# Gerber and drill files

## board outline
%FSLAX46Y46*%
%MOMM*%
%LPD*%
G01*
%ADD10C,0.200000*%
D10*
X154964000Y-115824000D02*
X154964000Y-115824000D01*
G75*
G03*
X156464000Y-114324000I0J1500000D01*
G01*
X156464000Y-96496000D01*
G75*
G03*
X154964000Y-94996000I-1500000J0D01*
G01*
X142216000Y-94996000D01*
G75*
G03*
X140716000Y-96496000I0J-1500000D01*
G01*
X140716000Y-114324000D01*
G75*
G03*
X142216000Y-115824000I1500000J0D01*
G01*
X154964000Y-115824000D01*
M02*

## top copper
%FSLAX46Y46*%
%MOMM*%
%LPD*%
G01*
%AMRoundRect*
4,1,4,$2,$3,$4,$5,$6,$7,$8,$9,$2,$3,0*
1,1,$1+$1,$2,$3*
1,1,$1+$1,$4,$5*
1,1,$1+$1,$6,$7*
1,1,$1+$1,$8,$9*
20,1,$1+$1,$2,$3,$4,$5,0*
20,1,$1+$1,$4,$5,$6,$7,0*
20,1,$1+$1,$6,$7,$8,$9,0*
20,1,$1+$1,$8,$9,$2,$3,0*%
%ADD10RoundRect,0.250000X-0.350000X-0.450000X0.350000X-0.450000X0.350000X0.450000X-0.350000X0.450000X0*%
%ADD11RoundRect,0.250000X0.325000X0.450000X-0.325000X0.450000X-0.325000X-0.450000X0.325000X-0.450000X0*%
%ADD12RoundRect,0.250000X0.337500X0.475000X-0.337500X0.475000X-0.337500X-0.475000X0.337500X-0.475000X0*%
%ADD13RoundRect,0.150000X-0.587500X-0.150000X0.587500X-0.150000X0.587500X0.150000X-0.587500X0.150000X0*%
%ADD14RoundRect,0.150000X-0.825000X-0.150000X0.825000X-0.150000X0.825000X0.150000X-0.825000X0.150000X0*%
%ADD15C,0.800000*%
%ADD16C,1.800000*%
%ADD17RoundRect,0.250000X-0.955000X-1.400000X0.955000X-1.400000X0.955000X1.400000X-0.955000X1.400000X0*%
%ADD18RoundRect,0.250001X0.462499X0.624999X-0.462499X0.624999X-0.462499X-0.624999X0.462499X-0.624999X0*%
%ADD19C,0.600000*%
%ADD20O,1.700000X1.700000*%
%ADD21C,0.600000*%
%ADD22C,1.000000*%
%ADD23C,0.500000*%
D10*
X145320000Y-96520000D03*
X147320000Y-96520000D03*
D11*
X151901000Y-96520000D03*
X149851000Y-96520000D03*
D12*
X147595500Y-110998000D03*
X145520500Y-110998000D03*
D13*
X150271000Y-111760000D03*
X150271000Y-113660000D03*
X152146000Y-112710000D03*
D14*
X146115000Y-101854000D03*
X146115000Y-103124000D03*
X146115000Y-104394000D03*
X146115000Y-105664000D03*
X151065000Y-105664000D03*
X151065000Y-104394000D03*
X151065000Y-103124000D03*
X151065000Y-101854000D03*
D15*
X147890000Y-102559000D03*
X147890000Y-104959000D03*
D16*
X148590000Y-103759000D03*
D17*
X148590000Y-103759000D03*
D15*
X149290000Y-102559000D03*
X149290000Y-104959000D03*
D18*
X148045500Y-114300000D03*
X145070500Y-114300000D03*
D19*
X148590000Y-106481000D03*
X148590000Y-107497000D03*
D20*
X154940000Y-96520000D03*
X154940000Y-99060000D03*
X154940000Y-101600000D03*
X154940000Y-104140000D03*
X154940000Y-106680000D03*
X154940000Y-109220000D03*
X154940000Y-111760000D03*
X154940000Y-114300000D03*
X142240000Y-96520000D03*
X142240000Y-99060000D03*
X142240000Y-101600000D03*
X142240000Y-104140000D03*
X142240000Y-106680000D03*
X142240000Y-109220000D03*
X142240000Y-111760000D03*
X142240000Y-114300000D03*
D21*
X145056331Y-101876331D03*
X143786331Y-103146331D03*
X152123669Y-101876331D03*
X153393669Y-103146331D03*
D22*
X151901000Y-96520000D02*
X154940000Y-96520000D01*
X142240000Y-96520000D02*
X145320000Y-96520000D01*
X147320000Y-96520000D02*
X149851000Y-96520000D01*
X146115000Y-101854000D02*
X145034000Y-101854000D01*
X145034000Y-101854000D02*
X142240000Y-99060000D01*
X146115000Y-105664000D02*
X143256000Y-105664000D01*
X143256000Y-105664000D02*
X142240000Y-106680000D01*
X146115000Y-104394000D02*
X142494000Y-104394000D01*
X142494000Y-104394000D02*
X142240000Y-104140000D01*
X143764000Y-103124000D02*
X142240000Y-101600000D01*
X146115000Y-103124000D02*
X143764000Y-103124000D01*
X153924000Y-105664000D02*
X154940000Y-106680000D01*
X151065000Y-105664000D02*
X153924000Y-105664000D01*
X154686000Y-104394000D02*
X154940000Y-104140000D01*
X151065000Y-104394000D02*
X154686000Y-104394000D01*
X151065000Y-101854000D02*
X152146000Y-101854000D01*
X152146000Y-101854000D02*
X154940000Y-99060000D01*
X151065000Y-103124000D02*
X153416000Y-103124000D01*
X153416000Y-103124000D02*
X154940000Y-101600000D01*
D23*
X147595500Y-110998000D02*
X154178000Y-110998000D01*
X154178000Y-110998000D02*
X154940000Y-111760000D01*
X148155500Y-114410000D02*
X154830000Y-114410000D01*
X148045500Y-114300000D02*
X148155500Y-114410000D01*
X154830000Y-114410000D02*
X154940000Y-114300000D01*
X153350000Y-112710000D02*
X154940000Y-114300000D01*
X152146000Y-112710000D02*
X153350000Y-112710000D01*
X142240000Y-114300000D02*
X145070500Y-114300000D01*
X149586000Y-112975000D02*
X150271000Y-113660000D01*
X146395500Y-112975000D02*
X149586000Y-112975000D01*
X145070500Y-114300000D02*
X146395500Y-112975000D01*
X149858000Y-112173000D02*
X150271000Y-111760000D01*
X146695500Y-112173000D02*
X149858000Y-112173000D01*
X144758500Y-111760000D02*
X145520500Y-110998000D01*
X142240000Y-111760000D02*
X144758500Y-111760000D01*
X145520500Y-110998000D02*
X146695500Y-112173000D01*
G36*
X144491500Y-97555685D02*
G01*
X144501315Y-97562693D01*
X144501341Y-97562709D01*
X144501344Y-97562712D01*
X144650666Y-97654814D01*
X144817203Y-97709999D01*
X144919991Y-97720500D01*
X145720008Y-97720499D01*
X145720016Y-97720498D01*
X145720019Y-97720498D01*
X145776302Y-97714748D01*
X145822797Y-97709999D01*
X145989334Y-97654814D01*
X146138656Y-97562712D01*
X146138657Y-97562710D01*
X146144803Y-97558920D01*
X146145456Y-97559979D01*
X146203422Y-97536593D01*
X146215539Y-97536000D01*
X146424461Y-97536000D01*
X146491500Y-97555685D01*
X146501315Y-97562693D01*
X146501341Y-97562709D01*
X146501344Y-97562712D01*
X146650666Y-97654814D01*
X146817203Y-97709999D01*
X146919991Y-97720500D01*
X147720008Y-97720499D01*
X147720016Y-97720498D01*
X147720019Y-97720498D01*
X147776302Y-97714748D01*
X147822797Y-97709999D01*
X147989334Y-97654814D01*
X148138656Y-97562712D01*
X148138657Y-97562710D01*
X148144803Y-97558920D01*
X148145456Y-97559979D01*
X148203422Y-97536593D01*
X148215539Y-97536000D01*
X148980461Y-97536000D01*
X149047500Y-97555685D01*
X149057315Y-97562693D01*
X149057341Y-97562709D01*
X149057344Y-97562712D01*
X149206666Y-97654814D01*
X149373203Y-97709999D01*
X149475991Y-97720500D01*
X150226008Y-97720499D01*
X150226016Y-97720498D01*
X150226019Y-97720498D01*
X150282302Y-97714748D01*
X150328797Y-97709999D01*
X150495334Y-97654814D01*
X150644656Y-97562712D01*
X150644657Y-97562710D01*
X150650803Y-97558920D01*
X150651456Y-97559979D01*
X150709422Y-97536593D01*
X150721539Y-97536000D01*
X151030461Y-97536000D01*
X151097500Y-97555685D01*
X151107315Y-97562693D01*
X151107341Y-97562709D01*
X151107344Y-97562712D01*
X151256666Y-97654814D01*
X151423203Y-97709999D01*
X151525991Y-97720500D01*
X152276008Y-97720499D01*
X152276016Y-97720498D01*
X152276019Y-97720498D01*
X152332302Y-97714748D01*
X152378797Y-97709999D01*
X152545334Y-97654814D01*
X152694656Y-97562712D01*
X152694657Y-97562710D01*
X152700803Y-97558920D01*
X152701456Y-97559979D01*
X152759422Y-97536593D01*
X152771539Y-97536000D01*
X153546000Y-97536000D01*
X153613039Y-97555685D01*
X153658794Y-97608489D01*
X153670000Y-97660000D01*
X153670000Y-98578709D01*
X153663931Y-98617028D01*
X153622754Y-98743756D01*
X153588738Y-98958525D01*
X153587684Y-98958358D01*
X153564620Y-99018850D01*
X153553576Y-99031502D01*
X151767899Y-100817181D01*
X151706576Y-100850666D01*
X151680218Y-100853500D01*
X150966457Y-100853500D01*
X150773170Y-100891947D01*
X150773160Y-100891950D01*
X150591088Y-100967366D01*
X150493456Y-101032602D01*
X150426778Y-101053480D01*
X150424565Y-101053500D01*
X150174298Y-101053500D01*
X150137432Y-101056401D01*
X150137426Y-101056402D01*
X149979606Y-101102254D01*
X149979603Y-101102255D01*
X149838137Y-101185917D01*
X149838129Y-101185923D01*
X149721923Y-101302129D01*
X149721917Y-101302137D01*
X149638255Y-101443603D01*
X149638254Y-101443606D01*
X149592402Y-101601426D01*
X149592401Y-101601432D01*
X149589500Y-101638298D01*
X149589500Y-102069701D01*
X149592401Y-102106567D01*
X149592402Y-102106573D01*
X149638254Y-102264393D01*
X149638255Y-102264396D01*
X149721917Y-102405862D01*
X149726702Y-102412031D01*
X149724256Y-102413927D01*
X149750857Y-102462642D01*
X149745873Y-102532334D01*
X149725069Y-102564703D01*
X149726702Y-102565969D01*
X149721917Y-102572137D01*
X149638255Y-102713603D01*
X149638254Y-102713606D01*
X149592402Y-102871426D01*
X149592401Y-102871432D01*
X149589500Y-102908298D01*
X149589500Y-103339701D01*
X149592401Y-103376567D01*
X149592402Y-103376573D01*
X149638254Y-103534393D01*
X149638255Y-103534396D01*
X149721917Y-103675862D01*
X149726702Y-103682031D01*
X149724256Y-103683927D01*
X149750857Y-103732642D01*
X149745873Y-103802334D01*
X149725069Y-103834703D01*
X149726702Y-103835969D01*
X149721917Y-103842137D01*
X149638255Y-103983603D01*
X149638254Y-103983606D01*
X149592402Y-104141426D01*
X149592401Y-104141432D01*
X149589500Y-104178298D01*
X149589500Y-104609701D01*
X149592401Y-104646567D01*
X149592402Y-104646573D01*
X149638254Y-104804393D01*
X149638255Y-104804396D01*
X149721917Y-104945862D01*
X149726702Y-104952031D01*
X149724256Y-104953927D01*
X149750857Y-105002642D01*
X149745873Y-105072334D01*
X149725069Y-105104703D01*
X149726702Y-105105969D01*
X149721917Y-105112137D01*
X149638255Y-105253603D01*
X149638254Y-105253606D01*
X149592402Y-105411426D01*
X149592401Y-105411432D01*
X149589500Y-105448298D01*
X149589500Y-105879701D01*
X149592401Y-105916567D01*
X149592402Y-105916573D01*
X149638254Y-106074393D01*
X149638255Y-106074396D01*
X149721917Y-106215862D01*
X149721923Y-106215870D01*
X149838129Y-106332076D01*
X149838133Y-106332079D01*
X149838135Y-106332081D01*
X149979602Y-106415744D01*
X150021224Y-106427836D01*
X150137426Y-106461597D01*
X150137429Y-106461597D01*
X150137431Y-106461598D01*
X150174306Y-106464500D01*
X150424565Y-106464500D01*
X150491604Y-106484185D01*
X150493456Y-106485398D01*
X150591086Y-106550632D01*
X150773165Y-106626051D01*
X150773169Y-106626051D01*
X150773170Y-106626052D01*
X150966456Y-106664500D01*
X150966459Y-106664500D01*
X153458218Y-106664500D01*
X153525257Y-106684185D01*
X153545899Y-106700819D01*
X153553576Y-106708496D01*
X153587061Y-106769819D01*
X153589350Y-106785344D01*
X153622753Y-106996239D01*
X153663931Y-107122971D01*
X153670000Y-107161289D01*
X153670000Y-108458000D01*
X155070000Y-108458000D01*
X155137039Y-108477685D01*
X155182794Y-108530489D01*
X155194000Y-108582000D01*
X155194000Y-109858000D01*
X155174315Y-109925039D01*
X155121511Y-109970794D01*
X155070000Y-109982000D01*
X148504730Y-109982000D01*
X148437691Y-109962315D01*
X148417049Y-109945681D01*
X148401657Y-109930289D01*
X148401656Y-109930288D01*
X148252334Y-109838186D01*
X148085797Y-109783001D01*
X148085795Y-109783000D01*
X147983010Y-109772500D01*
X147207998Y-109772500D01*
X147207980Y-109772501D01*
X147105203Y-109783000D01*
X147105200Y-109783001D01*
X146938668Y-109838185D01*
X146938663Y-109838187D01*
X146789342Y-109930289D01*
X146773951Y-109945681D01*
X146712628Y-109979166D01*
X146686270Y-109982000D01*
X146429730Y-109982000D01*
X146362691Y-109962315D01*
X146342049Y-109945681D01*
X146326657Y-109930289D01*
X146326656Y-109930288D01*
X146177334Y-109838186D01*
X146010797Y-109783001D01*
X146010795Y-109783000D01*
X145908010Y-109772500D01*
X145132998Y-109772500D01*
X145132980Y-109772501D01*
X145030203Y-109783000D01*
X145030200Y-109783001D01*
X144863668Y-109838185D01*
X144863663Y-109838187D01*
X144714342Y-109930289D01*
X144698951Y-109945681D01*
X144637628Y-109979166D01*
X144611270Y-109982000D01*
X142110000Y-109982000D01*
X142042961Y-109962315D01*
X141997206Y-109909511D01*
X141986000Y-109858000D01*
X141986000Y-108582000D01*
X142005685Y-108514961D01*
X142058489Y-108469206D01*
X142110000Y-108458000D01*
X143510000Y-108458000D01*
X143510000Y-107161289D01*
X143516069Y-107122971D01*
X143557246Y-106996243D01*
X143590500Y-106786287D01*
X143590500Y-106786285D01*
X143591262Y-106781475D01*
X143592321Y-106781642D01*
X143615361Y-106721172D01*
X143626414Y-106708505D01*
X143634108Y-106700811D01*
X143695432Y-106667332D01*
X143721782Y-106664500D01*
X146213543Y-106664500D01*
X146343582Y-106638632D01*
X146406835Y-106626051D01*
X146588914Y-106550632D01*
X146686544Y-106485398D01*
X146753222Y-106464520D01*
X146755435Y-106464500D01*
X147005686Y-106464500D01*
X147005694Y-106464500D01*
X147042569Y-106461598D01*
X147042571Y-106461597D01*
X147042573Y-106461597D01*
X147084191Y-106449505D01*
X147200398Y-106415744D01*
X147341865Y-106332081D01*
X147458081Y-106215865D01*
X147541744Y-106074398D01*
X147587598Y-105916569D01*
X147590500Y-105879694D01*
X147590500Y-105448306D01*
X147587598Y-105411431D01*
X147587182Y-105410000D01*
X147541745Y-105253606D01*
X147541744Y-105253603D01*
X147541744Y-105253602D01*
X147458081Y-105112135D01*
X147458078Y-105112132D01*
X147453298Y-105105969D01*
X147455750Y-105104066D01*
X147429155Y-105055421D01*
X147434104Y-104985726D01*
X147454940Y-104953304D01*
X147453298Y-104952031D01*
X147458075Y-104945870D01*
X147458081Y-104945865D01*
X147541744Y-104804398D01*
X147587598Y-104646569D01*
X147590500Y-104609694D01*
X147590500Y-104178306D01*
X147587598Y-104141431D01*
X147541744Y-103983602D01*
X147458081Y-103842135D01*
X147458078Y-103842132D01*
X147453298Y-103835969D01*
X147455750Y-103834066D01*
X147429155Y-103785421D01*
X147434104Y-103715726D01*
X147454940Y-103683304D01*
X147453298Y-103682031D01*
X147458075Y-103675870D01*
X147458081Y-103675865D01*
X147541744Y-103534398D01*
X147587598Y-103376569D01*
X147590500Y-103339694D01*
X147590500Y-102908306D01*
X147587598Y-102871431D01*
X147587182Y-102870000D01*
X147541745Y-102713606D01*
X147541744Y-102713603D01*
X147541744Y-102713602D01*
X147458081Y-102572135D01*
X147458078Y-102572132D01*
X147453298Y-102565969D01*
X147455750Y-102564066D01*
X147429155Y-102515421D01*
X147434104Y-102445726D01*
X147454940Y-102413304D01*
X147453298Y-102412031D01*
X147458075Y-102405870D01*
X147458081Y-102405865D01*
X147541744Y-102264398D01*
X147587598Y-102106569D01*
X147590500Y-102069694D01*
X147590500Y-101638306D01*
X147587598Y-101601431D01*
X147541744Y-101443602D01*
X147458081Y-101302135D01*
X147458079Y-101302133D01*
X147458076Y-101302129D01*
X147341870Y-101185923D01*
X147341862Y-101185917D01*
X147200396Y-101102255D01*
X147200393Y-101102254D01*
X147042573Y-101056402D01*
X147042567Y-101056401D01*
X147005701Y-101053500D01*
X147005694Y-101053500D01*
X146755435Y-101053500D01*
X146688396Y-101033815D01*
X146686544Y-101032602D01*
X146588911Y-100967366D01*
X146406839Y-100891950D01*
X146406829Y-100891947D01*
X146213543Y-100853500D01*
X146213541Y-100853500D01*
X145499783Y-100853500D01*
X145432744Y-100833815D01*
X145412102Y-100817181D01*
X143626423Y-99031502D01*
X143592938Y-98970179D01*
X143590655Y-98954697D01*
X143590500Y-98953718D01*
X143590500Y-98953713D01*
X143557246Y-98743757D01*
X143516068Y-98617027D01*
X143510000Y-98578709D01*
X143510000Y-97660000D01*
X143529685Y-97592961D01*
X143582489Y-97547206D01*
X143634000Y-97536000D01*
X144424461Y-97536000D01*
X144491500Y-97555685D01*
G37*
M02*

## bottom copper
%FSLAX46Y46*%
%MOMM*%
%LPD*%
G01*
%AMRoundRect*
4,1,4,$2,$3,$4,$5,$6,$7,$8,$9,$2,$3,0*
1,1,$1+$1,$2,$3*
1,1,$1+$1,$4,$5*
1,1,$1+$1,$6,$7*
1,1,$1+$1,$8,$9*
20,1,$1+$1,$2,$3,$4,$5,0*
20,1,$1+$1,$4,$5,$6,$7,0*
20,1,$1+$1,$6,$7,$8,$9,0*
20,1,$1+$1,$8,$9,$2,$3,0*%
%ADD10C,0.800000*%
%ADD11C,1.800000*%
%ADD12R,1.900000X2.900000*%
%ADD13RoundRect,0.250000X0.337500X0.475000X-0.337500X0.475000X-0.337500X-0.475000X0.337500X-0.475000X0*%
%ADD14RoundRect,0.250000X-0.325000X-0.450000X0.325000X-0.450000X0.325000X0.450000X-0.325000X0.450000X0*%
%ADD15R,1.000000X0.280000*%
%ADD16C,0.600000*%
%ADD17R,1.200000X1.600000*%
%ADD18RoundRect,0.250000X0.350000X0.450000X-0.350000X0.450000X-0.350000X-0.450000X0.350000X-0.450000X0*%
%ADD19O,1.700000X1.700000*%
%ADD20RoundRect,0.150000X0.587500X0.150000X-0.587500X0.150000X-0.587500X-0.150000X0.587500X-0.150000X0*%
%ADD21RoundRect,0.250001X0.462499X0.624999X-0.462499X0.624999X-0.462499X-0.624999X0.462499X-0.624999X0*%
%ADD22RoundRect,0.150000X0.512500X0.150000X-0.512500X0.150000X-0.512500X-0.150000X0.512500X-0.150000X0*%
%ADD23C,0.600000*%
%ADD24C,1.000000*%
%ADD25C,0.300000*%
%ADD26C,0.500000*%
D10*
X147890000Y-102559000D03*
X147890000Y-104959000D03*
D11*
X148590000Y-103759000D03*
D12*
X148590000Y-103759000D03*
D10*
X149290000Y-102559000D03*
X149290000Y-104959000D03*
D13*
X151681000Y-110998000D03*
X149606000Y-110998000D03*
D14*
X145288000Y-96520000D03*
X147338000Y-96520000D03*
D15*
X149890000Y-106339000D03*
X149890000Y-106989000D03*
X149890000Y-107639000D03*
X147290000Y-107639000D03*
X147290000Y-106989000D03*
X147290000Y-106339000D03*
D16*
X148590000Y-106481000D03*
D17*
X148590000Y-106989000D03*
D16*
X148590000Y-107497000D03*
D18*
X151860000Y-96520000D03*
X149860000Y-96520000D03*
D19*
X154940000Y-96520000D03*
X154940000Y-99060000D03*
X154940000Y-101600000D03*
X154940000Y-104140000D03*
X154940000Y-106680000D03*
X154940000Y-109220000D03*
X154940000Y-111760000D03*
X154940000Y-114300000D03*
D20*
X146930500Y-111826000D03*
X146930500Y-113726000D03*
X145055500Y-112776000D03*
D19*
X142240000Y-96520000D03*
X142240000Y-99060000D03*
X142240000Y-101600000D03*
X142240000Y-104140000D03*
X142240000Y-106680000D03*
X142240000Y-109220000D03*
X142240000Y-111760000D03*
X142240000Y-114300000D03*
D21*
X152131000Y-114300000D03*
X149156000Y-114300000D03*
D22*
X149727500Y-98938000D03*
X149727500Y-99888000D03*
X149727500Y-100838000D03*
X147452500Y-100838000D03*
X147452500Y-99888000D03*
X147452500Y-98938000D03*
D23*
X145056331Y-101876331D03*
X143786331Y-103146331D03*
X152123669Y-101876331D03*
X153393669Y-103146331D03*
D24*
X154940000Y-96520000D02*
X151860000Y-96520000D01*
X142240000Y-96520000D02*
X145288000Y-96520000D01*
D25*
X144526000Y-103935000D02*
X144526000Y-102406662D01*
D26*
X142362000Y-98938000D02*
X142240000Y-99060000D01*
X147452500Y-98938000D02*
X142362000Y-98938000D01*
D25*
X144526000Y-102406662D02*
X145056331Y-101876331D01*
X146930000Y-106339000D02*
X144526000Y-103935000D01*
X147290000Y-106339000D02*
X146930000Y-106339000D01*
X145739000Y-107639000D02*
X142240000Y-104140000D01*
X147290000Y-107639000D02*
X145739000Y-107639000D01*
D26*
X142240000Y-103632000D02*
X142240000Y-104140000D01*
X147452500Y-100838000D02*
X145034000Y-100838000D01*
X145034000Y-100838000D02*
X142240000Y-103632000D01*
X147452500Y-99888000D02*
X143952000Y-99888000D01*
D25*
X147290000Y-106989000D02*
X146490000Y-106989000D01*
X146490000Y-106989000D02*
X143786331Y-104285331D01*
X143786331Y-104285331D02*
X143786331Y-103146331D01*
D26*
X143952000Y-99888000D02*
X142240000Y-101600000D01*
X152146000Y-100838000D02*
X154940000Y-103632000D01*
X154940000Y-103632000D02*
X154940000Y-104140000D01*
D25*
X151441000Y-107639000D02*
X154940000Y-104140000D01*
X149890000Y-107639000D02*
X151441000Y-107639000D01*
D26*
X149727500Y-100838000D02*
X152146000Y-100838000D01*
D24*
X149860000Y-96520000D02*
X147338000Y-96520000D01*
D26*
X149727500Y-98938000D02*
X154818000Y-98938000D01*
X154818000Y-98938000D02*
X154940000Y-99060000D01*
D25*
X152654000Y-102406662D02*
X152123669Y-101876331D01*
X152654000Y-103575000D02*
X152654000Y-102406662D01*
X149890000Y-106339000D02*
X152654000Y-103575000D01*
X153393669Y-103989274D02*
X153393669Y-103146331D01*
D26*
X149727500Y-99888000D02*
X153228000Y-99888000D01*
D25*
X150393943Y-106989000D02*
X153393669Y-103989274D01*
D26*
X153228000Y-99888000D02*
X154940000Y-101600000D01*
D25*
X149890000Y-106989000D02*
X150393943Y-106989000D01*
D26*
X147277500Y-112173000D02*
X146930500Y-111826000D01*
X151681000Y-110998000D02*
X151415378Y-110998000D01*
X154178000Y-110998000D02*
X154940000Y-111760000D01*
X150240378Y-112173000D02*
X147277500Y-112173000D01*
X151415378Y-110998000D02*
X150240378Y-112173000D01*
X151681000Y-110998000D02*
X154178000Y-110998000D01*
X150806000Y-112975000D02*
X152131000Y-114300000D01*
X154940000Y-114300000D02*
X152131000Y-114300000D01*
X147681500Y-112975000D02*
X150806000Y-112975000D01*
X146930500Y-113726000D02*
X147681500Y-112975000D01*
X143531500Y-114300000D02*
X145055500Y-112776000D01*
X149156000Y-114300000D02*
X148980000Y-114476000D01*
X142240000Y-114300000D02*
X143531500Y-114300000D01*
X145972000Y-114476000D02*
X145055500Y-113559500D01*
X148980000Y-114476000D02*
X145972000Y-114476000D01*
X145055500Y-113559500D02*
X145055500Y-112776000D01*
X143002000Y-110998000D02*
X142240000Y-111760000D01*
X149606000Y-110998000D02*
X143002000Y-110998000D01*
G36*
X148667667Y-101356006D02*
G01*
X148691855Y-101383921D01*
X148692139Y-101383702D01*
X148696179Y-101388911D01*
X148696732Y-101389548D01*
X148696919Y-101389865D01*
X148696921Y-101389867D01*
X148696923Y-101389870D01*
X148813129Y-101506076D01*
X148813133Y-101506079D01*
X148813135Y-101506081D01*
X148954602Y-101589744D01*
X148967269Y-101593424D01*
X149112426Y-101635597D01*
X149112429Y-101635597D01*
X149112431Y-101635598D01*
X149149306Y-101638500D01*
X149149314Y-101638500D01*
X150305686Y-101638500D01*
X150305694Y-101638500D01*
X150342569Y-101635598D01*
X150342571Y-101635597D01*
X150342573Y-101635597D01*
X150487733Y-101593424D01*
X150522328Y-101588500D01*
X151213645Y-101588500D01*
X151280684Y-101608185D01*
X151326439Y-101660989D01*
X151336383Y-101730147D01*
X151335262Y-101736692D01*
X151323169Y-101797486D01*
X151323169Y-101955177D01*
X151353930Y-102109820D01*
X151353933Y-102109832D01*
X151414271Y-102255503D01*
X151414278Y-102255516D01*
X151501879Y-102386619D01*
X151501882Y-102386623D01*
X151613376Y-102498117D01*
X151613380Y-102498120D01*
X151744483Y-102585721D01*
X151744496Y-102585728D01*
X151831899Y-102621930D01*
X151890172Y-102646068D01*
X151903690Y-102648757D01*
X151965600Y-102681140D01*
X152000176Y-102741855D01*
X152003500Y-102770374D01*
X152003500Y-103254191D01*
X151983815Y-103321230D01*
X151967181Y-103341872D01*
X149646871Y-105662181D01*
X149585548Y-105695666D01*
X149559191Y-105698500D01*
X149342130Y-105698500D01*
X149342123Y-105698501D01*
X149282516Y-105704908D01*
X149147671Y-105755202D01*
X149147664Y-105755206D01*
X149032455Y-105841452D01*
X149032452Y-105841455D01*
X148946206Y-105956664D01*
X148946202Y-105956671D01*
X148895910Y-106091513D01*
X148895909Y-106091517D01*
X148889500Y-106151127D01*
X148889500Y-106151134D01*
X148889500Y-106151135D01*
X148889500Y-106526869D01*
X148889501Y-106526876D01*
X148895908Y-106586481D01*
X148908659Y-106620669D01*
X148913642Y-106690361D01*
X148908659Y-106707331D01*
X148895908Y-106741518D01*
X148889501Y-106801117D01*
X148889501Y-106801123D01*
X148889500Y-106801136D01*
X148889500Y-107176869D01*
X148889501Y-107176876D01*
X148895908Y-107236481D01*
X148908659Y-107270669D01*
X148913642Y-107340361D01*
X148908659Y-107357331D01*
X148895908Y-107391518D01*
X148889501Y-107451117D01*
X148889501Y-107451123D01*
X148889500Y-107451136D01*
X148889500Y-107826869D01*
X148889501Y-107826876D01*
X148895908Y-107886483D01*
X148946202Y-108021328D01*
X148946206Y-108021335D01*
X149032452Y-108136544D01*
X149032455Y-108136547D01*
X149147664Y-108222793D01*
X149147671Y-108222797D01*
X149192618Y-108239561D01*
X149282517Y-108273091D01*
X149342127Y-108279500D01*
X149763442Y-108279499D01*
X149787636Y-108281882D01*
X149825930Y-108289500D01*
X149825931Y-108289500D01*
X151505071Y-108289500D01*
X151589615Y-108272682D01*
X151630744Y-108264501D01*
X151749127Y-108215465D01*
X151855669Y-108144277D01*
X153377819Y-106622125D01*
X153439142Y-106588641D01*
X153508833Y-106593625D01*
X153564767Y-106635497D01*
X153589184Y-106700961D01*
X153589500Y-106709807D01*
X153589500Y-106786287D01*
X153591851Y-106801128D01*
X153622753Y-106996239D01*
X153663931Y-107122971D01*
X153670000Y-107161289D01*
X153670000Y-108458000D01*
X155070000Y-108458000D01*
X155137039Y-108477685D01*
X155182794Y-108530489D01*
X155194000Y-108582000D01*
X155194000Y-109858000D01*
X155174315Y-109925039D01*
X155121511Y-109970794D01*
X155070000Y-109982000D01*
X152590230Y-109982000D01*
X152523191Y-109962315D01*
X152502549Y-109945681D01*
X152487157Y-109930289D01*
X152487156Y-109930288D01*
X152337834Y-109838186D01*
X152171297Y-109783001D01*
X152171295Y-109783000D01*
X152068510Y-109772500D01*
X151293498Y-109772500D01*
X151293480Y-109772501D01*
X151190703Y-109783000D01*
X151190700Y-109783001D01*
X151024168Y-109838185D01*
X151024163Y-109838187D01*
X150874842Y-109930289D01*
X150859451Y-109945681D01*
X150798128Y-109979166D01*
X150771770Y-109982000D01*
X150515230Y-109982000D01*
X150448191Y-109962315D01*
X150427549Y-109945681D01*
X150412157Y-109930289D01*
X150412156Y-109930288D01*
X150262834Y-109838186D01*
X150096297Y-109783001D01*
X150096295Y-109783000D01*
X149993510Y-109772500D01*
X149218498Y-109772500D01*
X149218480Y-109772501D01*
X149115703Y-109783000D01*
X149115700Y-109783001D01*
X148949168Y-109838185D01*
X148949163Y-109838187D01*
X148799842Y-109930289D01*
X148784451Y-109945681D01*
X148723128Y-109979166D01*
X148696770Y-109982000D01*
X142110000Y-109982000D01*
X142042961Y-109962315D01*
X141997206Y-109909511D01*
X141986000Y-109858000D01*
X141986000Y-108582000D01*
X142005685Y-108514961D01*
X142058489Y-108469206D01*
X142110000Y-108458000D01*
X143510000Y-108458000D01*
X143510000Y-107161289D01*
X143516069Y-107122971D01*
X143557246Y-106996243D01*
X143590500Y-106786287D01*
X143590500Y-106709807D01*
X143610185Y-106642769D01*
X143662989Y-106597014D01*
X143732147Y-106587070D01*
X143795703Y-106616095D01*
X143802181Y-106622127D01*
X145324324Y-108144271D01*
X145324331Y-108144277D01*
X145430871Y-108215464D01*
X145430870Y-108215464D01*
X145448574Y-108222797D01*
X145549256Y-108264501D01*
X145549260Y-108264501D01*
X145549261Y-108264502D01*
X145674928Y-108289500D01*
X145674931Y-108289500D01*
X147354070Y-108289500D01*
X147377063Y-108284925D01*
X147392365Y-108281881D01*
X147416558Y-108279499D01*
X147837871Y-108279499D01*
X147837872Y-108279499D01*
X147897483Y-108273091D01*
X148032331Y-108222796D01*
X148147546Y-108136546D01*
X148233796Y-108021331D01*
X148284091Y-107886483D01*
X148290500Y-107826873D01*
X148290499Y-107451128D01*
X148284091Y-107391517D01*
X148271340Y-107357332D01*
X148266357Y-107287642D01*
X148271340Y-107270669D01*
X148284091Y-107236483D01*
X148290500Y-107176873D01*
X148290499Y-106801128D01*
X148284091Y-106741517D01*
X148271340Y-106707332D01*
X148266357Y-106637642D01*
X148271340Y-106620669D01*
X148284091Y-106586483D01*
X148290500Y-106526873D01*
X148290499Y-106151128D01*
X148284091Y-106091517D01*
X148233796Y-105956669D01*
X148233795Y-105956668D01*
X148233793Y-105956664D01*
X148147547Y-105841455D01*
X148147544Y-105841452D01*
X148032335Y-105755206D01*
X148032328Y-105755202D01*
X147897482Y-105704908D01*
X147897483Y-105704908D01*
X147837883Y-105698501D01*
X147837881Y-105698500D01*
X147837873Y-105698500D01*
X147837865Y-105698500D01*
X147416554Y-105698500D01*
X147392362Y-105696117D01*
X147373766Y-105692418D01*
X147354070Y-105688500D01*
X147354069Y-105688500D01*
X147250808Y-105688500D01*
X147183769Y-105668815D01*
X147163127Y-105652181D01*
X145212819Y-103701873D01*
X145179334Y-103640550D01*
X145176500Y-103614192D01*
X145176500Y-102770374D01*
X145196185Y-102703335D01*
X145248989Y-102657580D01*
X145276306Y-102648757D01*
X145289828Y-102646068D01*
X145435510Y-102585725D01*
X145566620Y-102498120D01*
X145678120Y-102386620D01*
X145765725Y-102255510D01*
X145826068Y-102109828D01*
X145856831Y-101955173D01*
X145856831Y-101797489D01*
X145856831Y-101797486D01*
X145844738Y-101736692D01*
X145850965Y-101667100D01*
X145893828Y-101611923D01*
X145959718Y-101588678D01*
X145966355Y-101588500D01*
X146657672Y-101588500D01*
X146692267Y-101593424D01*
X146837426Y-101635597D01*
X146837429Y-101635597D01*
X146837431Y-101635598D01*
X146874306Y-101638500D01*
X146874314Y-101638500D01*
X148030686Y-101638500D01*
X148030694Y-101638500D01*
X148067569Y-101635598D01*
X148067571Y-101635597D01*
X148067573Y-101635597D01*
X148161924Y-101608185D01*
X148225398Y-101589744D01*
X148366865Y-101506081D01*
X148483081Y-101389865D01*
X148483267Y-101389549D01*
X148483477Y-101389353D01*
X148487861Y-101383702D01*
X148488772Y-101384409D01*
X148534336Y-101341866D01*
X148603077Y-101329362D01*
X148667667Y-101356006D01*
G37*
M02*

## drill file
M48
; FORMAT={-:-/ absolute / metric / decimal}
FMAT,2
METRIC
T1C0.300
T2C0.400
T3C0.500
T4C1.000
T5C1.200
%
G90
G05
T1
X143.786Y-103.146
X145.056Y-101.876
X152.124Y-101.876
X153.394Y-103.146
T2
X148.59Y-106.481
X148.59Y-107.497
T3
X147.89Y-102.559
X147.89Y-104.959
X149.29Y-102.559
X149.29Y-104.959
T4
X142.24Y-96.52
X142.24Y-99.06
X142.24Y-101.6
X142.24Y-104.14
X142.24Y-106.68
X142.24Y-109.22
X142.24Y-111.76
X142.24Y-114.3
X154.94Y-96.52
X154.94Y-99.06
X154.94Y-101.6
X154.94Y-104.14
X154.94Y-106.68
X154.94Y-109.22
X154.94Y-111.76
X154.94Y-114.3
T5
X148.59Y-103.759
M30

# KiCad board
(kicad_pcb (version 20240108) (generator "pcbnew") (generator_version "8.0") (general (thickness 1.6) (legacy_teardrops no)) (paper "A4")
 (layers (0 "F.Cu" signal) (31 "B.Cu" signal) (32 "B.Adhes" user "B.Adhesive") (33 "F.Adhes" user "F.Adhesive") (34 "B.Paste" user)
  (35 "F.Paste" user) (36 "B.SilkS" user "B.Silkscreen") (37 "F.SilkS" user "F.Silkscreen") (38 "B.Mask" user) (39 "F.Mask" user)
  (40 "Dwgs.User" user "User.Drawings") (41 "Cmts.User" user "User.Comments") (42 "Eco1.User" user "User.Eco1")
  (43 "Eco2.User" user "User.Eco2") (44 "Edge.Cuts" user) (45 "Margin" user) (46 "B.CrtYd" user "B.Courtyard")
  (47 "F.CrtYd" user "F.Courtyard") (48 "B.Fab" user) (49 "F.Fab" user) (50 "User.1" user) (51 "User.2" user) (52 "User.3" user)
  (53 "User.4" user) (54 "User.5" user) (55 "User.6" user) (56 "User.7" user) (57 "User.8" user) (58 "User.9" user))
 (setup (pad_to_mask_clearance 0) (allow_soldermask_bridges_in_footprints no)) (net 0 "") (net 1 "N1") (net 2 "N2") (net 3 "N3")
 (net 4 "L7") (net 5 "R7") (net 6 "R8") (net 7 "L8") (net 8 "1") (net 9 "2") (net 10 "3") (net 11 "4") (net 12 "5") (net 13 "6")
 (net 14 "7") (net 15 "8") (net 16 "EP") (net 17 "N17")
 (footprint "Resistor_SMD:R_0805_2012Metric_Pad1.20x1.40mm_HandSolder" (layer "F.Cu") (at 146.32 96.52)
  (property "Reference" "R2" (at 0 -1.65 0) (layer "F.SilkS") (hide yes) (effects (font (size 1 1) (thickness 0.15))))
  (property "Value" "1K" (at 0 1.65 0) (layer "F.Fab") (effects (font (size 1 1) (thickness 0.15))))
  (pad "1" smd roundrect (at -1 0) (size 1.2 1.4) (layers "F.Cu" "F.Paste" "F.Mask") (roundrect_rratio 0.208333) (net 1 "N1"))
  (pad "2" smd roundrect (at 1 0) (size 1.2 1.4) (layers "F.Cu" "F.Paste" "F.Mask") (roundrect_rratio 0.208333) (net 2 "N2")))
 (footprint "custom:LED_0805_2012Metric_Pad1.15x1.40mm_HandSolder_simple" (layer "F.Cu") (at 150.876 96.52 180)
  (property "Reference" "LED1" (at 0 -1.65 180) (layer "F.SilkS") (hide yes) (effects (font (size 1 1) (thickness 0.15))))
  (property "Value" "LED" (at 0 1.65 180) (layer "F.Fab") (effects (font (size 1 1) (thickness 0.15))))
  (pad "1" smd roundrect (at -1.025 0 180) (size 1.15 1.4) (layers "F.Cu" "F.Paste" "F.Mask") (roundrect_rratio 0.217391) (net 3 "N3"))
  (pad "2" smd roundrect (at 1.025 0 180) (size 1.15 1.4) (layers "F.Cu" "F.Paste" "F.Mask") (roundrect_rratio 0.217391) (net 2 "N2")))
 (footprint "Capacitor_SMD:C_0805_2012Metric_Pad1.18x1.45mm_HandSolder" (layer "F.Cu") (at 146.558 110.998 180)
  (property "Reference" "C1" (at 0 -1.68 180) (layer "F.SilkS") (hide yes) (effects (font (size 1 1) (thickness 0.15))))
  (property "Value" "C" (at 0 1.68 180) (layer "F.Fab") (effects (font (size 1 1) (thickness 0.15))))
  (pad "1" smd roundrect (at -1.0375 0 180) (size 1.175 1.45) (layers "F.Cu" "F.Paste" "F.Mask") (roundrect_rratio 0.212766) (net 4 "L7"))
  (pad "2" smd roundrect (at 1.0375 0 180) (size 1.175 1.45) (layers "F.Cu" "F.Paste" "F.Mask") (roundrect_rratio 0.212766) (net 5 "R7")))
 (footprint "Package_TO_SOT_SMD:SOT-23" (layer "F.Cu") (at 151.2085 112.71)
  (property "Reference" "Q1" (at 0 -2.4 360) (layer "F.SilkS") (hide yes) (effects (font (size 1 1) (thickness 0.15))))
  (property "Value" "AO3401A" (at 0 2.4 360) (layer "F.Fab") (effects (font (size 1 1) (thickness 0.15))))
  (pad "1" smd roundrect (at -0.9375 -0.95) (size 1.475 0.6) (layers "F.Cu" "F.Paste" "F.Mask") (roundrect_rratio 0.25) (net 5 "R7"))
  (pad "2" smd roundrect (at -0.9375 0.95) (size 1.475 0.6) (layers "F.Cu" "F.Paste" "F.Mask") (roundrect_rratio 0.25) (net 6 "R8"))
  (pad "3" smd roundrect (at 0.9375 0) (size 1.475 0.6) (layers "F.Cu" "F.Paste" "F.Mask") (roundrect_rratio 0.25) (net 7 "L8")))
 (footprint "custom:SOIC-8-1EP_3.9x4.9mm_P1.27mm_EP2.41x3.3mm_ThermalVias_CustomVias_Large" (layer "F.Cu") (at 148.59 103.759)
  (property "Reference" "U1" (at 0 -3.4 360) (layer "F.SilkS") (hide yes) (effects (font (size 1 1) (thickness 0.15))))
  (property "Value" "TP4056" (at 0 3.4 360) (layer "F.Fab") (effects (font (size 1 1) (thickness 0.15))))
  (pad "" smd roundrect (at -0.6 -0.825) (size 1.01 1.38) (layers "F.Paste") (roundrect_rratio 0.247525))
  (pad "" smd roundrect (at -0.6 0.825) (size 1.01 1.38) (layers "F.Paste") (roundrect_rratio 0.247525))
  (pad "" smd roundrect (at 0.6 -0.825) (size 1.01 1.38) (layers "F.Paste") (roundrect_rratio 0.247525))
  (pad "" smd roundrect (at 0.6 0.825) (size 1.01 1.38) (layers "F.Paste") (roundrect_rratio 0.247525))
  (pad "1" smd roundrect (at -2.475 -1.905) (size 1.95 0.6) (layers "F.Cu" "F.Paste" "F.Mask") (roundrect_rratio 0.25) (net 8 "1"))
  (pad "2" smd roundrect (at -2.475 -0.635) (size 1.95 0.6) (layers "F.Cu" "F.Paste" "F.Mask") (roundrect_rratio 0.25) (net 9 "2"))
  (pad "3" smd roundrect (at -2.475 0.635) (size 1.95 0.6) (layers "F.Cu" "F.Paste" "F.Mask") (roundrect_rratio 0.25) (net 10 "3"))
  (pad "4" smd roundrect (at -2.475 1.905) (size 1.95 0.6) (layers "F.Cu" "F.Paste" "F.Mask") (roundrect_rratio 0.25) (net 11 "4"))
  (pad "5" smd roundrect (at 2.475 1.905) (size 1.95 0.6) (layers "F.Cu" "F.Paste" "F.Mask") (roundrect_rratio 0.25) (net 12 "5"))
  (pad "6" smd roundrect (at 2.475 0.635) (size 1.95 0.6) (layers "F.Cu" "F.Paste" "F.Mask") (roundrect_rratio 0.25) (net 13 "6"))
  (pad "7" smd roundrect (at 2.475 -0.635) (size 1.95 0.6) (layers "F.Cu" "F.Paste" "F.Mask") (roundrect_rratio 0.25) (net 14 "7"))
  (pad "8" smd roundrect (at 2.475 -1.905) (size 1.95 0.6) (layers "F.Cu" "F.Paste" "F.Mask") (roundrect_rratio 0.25) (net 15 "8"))
  (pad "9" thru_hole circle (at -0.7 -1.2) (size 0.8 0.8) (drill 0.5) (layers "*.Cu") (remove_unused_layers no) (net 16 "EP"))
  (pad "9" thru_hole circle (at -0.7 1.2) (size 0.8 0.8) (drill 0.5) (layers "*.Cu") (remove_unused_layers no) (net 16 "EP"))
  (pad "9" thru_hole circle (at 0 0) (size 1.8 1.8) (drill 1.2) (layers "*.Cu") (remove_unused_layers no) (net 16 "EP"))
  (pad "9" smd rect (at 0 0) (size 1.9 2.9) (layers "B.Cu") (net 16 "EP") (zone_connect 2))
  (pad "9" smd roundrect (at 0 0) (size 2.41 3.3) (layers "F.Cu" "F.Mask") (roundrect_rratio 0.1037344398) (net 16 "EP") (zone_connect 2))
  (pad "9" thru_hole circle (at 0.7 -1.2) (size 0.8 0.8) (drill 0.5) (layers "*.Cu") (remove_unused_layers no) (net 16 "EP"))
  (pad "9" thru_hole circle (at 0.7 1.2) (size 0.8 0.8) (drill 0.5) (layers "*.Cu") (remove_unused_layers no) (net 16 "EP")))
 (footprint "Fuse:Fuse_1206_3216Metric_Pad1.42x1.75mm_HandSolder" (layer "F.Cu") (at 146.558 114.3 180)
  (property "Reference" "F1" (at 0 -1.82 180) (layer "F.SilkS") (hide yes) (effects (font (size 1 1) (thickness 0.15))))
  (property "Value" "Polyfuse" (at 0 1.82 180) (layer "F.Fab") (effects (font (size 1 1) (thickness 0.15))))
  (pad "1" smd roundrect (at -1.4875 0 180) (size 1.425 1.75) (layers "F.Cu" "F.Paste" "F.Mask") (roundrect_rratio 0.175439) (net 7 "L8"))
  (pad "2" smd roundrect (at 1.4875 0 180) (size 1.425 1.75) (layers "F.Cu" "F.Paste" "F.Mask") (roundrect_rratio 0.175439) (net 6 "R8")))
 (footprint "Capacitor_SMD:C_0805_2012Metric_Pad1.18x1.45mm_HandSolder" (layer "B.Cu") (at 150.6435 110.998 180)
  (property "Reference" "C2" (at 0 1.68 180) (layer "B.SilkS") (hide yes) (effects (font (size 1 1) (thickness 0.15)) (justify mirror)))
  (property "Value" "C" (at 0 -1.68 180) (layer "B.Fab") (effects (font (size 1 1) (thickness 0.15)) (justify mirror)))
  (pad "1" smd roundrect (at -1.0375 0 180) (size 1.175 1.45) (layers "B.Cu" "B.Paste" "B.Mask") (roundrect_rratio 0.212766) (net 4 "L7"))
  (pad "2" smd roundrect (at 1.0375 0 180) (size 1.175 1.45) (layers "B.Cu" "B.Paste" "B.Mask") (roundrect_rratio 0.212766) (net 5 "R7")))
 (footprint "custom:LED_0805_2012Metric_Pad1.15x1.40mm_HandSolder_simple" (layer "B.Cu") (at 146.313 96.52)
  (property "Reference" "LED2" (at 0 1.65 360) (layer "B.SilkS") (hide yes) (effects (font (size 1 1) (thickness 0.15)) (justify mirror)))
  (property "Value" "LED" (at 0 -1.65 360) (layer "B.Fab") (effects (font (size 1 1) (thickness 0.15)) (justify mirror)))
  (pad "1" smd roundrect (at -1.025 0) (size 1.15 1.4) (layers "B.Cu" "B.Paste" "B.Mask") (roundrect_rratio 0.217391) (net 1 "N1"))
  (pad "2" smd roundrect (at 1.025 0) (size 1.15 1.4) (layers "B.Cu" "B.Paste" "B.Mask") (roundrect_rratio 0.217391) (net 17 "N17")))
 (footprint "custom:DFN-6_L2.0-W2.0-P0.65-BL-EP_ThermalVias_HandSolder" (layer "B.Cu") (at 148.59 106.989 -90)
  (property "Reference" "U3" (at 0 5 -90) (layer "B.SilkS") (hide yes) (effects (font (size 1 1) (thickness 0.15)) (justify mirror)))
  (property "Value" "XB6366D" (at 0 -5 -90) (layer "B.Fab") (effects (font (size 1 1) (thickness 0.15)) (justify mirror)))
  (pad "1" smd rect (at -0.65 -1.3 270) (size 0.28 1) (layers "B.Cu" "B.Paste" "B.Mask") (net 15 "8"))
  (pad "2" smd rect (at 0 -1.3 270) (size 0.28 1) (layers "B.Cu" "B.Paste" "B.Mask") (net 14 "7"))
  (pad "3" smd rect (at 0.65 -1.3 270) (size 0.28 1) (layers "B.Cu" "B.Paste" "B.Mask") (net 13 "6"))
  (pad "4" smd rect (at 0.65 1.3 270) (size 0.28 1) (layers "B.Cu" "B.Paste" "B.Mask") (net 10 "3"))
  (pad "5" smd rect (at 0 1.3 270) (size 0.28 1) (layers "B.Cu" "B.Paste" "B.Mask") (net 9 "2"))
  (pad "6" smd rect (at -0.65 1.3 270) (size 0.28 1) (layers "B.Cu" "B.Paste" "B.Mask") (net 8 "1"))
  (pad "7" thru_hole circle (at -0.508 0 270) (size 0.6 0.6) (drill 0.4) (layers "*.Cu") (remove_unused_layers no) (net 16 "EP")
   (solder_mask_margin 0.148) (clearance 0.5))
  (pad "7" smd rect (at 0 0 270) (size 1.6 1.2) (layers "B.Cu" "B.Paste" "B.Mask") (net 16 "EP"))
  (pad "7" thru_hole circle (at 0.508 0 270) (size 0.6 0.6) (drill 0.4) (layers "*.Cu") (remove_unused_layers no) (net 16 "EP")
   (solder_mask_margin 0.148) (clearance 0.5)))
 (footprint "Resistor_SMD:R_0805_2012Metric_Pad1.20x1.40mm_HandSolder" (layer "B.Cu") (at 150.86 96.52 180)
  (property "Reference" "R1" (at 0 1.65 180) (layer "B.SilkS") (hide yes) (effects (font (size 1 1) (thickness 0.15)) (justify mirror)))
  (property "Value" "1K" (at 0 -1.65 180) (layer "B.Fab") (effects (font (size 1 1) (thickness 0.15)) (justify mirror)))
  (pad "1" smd roundrect (at -1 0 180) (size 1.2 1.4) (layers "B.Cu" "B.Paste" "B.Mask") (roundrect_rratio 0.208333) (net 3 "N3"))
  (pad "2" smd roundrect (at 1 0 180) (size 1.2 1.4) (layers "B.Cu" "B.Paste" "B.Mask") (roundrect_rratio 0.208333) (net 17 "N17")))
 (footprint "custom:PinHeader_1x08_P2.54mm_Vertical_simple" (layer "B.Cu") (at 154.94 96.52 180)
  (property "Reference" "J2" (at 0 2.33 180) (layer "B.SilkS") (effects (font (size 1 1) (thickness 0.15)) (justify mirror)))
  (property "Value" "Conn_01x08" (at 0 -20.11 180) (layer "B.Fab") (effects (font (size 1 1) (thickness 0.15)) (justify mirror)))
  (pad "1" thru_hole oval (at 0 0 180) (size 1.7 1.7) (drill 1) (layers "*.Cu" "*.Mask") (remove_unused_layers no) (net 3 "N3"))
  (pad "2" thru_hole oval (at 0 -2.54 180) (size 1.7 1.7) (drill 1) (layers "*.Cu" "*.Mask") (remove_unused_layers no) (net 15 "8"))
  (pad "3" thru_hole oval (at 0 -5.08 180) (size 1.7 1.7) (drill 1) (layers "*.Cu" "*.Mask") (remove_unused_layers no) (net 14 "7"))
  (pad "4" thru_hole oval (at 0 -7.62 180) (size 1.7 1.7) (drill 1) (layers "*.Cu" "*.Mask") (remove_unused_layers no) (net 13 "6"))
  (pad "5" thru_hole oval (at 0 -10.16 180) (size 1.7 1.7) (drill 1) (layers "*.Cu" "*.Mask") (remove_unused_layers no) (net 12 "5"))
  (pad "6" thru_hole oval (at 0 -12.7 180) (size 1.7 1.7) (drill 1) (layers "*.Cu" "*.Mask") (remove_unused_layers no) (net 16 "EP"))
  (pad "7" thru_hole oval (at 0 -15.24 180) (size 1.7 1.7) (drill 1) (layers "*.Cu" "*.Mask") (remove_unused_layers no) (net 4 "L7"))
  (pad "8" thru_hole oval (at 0 -17.78 180) (size 1.7 1.7) (drill 1) (layers "*.Cu" "*.Mask") (remove_unused_layers no) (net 7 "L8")))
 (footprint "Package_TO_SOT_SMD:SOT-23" (layer "B.Cu") (at 145.993 112.776 180)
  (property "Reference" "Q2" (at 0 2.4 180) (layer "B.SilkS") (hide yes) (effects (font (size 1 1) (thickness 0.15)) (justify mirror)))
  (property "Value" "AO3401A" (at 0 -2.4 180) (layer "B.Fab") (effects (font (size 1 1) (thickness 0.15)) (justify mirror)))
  (pad "1" smd roundrect (at -0.9375 0.95 180) (size 1.475 0.6) (layers "B.Cu" "B.Paste" "B.Mask") (roundrect_rratio 0.25) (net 4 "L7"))
  (pad "2" smd roundrect (at -0.9375 -0.95 180) (size 1.475 0.6) (layers "B.Cu" "B.Paste" "B.Mask") (roundrect_rratio 0.25) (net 7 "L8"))
  (pad "3" smd roundrect (at 0.9375 0 180) (size 1.475 0.6) (layers "B.Cu" "B.Paste" "B.Mask") (roundrect_rratio 0.25) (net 6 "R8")))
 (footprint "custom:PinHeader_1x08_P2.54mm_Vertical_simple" (layer "B.Cu") (at 142.24 96.52 180)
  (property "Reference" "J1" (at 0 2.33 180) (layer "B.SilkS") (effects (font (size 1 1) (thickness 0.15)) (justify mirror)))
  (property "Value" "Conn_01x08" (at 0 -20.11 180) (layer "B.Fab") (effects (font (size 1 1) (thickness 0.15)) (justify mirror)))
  (pad "1" thru_hole oval (at 0 0 180) (size 1.7 1.7) (drill 1) (layers "*.Cu" "*.Mask") (remove_unused_layers no) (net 1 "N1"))
  (pad "2" thru_hole oval (at 0 -2.54 180) (size 1.7 1.7) (drill 1) (layers "*.Cu" "*.Mask") (remove_unused_layers no) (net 8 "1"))
  (pad "3" thru_hole oval (at 0 -5.08 180) (size 1.7 1.7) (drill 1) (layers "*.Cu" "*.Mask") (remove_unused_layers no) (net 9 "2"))
  (pad "4" thru_hole oval (at 0 -7.62 180) (size 1.7 1.7) (drill 1) (layers "*.Cu" "*.Mask") (remove_unused_layers no) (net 10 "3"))
  (pad "5" thru_hole oval (at 0 -10.16 180) (size 1.7 1.7) (drill 1) (layers "*.Cu" "*.Mask") (remove_unused_layers no) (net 11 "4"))
  (pad "6" thru_hole oval (at 0 -12.7 180) (size 1.7 1.7) (drill 1) (layers "*.Cu" "*.Mask") (remove_unused_layers no) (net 16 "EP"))
  (pad "7" thru_hole oval (at 0 -15.24 180) (size 1.7 1.7) (drill 1) (layers "*.Cu" "*.Mask") (remove_unused_layers no) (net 5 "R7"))
  (pad "8" thru_hole oval (at 0 -17.78 180) (size 1.7 1.7) (drill 1) (layers "*.Cu" "*.Mask") (remove_unused_layers no) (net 6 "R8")))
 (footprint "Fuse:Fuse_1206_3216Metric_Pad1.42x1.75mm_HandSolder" (layer "B.Cu") (at 150.6435 114.3 180)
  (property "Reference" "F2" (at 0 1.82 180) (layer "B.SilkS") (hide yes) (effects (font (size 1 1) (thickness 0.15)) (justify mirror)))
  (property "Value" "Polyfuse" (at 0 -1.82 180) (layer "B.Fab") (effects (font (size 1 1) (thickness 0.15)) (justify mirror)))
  (pad "1" smd roundrect (at -1.4875 0 180) (size 1.425 1.75) (layers "B.Cu" "B.Paste" "B.Mask") (roundrect_rratio 0.175439) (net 7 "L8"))
  (pad "2" smd roundrect (at 1.4875 0 180) (size 1.425 1.75) (layers "B.Cu" "B.Paste" "B.Mask") (roundrect_rratio 0.175439) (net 6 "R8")))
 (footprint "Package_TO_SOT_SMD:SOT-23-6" (layer "B.Cu") (at 148.59 99.888 180)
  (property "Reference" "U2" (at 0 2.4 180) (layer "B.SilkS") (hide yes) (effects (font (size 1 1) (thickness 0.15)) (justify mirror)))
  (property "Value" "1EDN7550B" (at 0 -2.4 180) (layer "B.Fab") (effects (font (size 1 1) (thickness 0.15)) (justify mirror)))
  (pad "1" smd roundrect (at -1.1375 0.95 180) (size 1.325 0.6) (layers "B.Cu" "B.Paste" "B.Mask") (roundrect_rratio 0.25) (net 15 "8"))
  (pad "2" smd roundrect (at -1.1375 0 180) (size 1.325 0.6) (layers "B.Cu" "B.Paste" "B.Mask") (roundrect_rratio 0.25) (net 14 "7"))
  (pad "3" smd roundrect (at -1.1375 -0.95 180) (size 1.325 0.6) (layers "B.Cu" "B.Paste" "B.Mask") (roundrect_rratio 0.25) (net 13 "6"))
  (pad "4" smd roundrect (at 1.1375 -0.95 180) (size 1.325 0.6) (layers "B.Cu" "B.Paste" "B.Mask") (roundrect_rratio 0.25) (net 10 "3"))
  (pad "5" smd roundrect (at 1.1375 0 180) (size 1.325 0.6) (layers "B.Cu" "B.Paste" "B.Mask") (roundrect_rratio 0.25) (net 9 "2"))
  (pad "6" smd roundrect (at 1.1375 0.95 180) (size 1.325 0.6) (layers "B.Cu" "B.Paste" "B.Mask") (roundrect_rratio 0.25) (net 8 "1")))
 (gr_poly
  (pts
   (arc (start 154.964 115.824) (mid 156.02466 115.38466) (end 156.464 114.324))
   (arc (start 156.464 96.496) (mid 156.02466 95.43534) (end 154.964 94.996))
   (arc (start 142.216 94.996) (mid 141.15534 95.43534) (end 140.716 96.496))
   (arc (start 140.716 114.324) (mid 141.15534 115.38466) (end 142.216 115.824)))
  (stroke (width 0.2) (type solid)) (fill none) (layer "Edge.Cuts"))
 (segment (start 151.901 96.52) (end 154.94 96.52) (width 1) (layer "F.Cu") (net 3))
 (segment (start 154.94 96.52) (end 151.86 96.52) (width 1) (layer "B.Cu") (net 3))
 (segment (start 142.24 96.52) (end 145.32 96.52) (width 1) (layer "F.Cu") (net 1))
 (segment (start 142.24 96.52) (end 145.288 96.52) (width 1) (layer "B.Cu") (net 1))
 (segment (start 147.32 96.52) (end 149.851 96.52) (width 1) (layer "F.Cu") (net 2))
 (segment (start 146.115 101.854) (end 145.034 101.854) (width 1) (layer "F.Cu") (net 8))
 (segment (start 145.034 101.854) (end 142.24 99.06) (width 1) (layer "F.Cu") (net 8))
 (via (at 145.056331 101.876331) (size 0.6) (drill 0.3) (layers "F.Cu" "B.Cu") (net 8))
 (segment (start 144.526 103.935) (end 144.526 102.406662) (width 0.3) (layer "B.Cu") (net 8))
 (segment (start 142.362 98.938) (end 142.24 99.06) (width 0.5) (layer "B.Cu") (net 8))
 (segment (start 147.4525 98.938) (end 142.362 98.938) (width 0.5) (layer "B.Cu") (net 8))
 (segment (start 144.526 102.406662) (end 145.056331 101.876331) (width 0.3) (layer "B.Cu") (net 8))
 (segment (start 146.93 106.339) (end 144.526 103.935) (width 0.3) (layer "B.Cu") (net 8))
 (segment (start 147.29 106.339) (end 146.93 106.339) (width 0.3) (layer "B.Cu") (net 8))
 (segment (start 146.115 105.664) (end 143.256 105.664) (width 1) (layer "F.Cu") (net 11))
 (segment (start 143.256 105.664) (end 142.24 106.68) (width 1) (layer "F.Cu") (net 11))
 (segment (start 146.115 104.394) (end 142.494 104.394) (width 1) (layer "F.Cu") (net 10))
 (segment (start 142.494 104.394) (end 142.24 104.14) (width 1) (layer "F.Cu") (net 10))
 (segment (start 145.739 107.639) (end 142.24 104.14) (width 0.3) (layer "B.Cu") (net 10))
 (segment (start 147.29 107.639) (end 145.739 107.639) (width 0.3) (layer "B.Cu") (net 10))
 (segment (start 142.24 103.632) (end 142.24 104.14) (width 0.5) (layer "B.Cu") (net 10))
 (segment (start 147.4525 100.838) (end 145.034 100.838) (width 0.5) (layer "B.Cu") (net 10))
 (segment (start 145.034 100.838) (end 142.24 103.632) (width 0.5) (layer "B.Cu") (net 10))
 (segment (start 143.764 103.124) (end 142.24 101.6) (width 1) (layer "F.Cu") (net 9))
 (segment (start 146.115 103.124) (end 143.764 103.124) (width 1) (layer "F.Cu") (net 9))
 (via (at 143.786331 103.146331) (size 0.6) (drill 0.3) (layers "F.Cu" "B.Cu") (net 9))
 (segment (start 147.4525 99.888) (end 143.952 99.888) (width 0.5) (layer "B.Cu") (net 9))
 (segment (start 147.29 106.989) (end 146.49 106.989) (width 0.3) (layer "B.Cu") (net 9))
 (segment (start 146.49 106.989) (end 143.786331 104.285331) (width 0.3) (layer "B.Cu") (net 9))
 (segment (start 143.786331 104.285331) (end 143.786331 103.146331) (width 0.3) (layer "B.Cu") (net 9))
 (segment (start 143.952 99.888) (end 142.24 101.6) (width 0.5) (layer "B.Cu") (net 9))
 (segment (start 153.924 105.664) (end 154.94 106.68) (width 1) (layer "F.Cu") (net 12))
 (segment (start 151.065 105.664) (end 153.924 105.664) (width 1) (layer "F.Cu") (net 12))
 (segment (start 154.686 104.394) (end 154.94 104.14) (width 1) (layer "F.Cu") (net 13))
 (segment (start 151.065 104.394) (end 154.686 104.394) (width 1) (layer "F.Cu") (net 13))
 (segment (start 152.146 100.838) (end 154.94 103.632) (width 0.5) (layer "B.Cu") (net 13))
 (segment (start 154.94 103.632) (end 154.94 104.14) (width 0.5) (layer "B.Cu") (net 13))
 (segment (start 151.441 107.639) (end 154.94 104.14) (width 0.3) (layer "B.Cu") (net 13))
 (segment (start 149.89 107.639) (end 151.441 107.639) (width 0.3) (layer "B.Cu") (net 13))
 (segment (start 149.7275 100.838) (end 152.146 100.838) (width 0.5) (layer "B.Cu") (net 13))
 (segment (start 149.86 96.52) (end 147.338 96.52) (width 1) (layer "B.Cu") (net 17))
 (segment (start 151.065 101.854) (end 152.146 101.854) (width 1) (layer "F.Cu") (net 15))
 (segment (start 152.146 101.854) (end 154.94 99.06) (width 1) (layer "F.Cu") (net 15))
 (via (at 152.123669 101.876331) (size 0.6) (drill 0.3) (layers "F.Cu" "B.Cu") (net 15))
 (segment (start 149.7275 98.938) (end 154.818 98.938) (width 0.5) (layer "B.Cu") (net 15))
 (segment (start 154.818 98.938) (end 154.94 99.06) (width 0.5) (layer "B.Cu") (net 15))
 (segment (start 152.654 102.406662) (end 152.123669 101.876331) (width 0.3) (layer "B.Cu") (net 15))
 (segment (start 152.654 103.575) (end 152.654 102.406662) (width 0.3) (layer "B.Cu") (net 15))
 (segment (start 149.89 106.339) (end 152.654 103.575) (width 0.3) (layer "B.Cu") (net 15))
 (segment (start 151.065 103.124) (end 153.416 103.124) (width 1) (layer "F.Cu") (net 14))
 (segment (start 153.416 103.124) (end 154.94 101.6) (width 1) (layer "F.Cu") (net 14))
 (via (at 153.393669 103.146331) (size 0.6) (drill 0.3) (layers "F.Cu" "B.Cu") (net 14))
 (segment (start 153.393669 103.989274) (end 153.393669 103.146331) (width 0.3) (layer "B.Cu") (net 14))
 (segment (start 149.7275 99.888) (end 153.228 99.888) (width 0.5) (layer "B.Cu") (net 14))
 (segment (start 150.393943 106.989) (end 153.393669 103.989274) (width 0.3) (layer "B.Cu") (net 14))
 (segment (start 153.228 99.888) (end 154.94 101.6) (width 0.5) (layer "B.Cu") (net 14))
 (segment (start 149.89 106.989) (end 150.393943 106.989) (width 0.3) (layer "B.Cu") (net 14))
 (segment (start 147.5955 110.998) (end 154.178 110.998) (width 0.5) (layer "F.Cu") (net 4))
 (segment (start 154.178 110.998) (end 154.94 111.76) (width 0.5) (layer "F.Cu") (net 4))
 (segment (start 147.2775 112.173) (end 146.9305 111.826) (width 0.5) (layer "B.Cu") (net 4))
 (segment (start 151.681 110.998) (end 151.415378 110.998) (width 0.5) (layer "B.Cu") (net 4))
 (segment (start 154.178 110.998) (end 154.94 111.76) (width 0.5) (layer "B.Cu") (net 4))
 (segment (start 150.240378 112.173) (end 147.2775 112.173) (width 0.5) (layer "B.Cu") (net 4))
 (segment (start 151.415378 110.998) (end 150.240378 112.173) (width 0.5) (layer "B.Cu") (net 4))
 (segment (start 151.681 110.998) (end 154.178 110.998) (width 0.5) (layer "B.Cu") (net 4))
 (segment (start 148.1555 114.41) (end 154.83 114.41) (width 0.5) (layer "F.Cu") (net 7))
 (segment (start 148.0455 114.3) (end 148.1555 114.41) (width 0.5) (layer "F.Cu") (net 7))
 (segment (start 154.83 114.41) (end 154.94 114.3) (width 0.5) (layer "F.Cu") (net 7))
 (segment (start 153.35 112.71) (end 154.94 114.3) (width 0.5) (layer "F.Cu") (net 7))
 (segment (start 152.146 112.71) (end 153.35 112.71) (width 0.5) (layer "F.Cu") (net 7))
 (segment (start 150.806 112.975) (end 152.131 114.3) (width 0.5) (layer "B.Cu") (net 7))
 (segment (start 154.94 114.3) (end 152.131 114.3) (width 0.5) (layer "B.Cu") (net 7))
 (segment (start 147.6815 112.975) (end 150.806 112.975) (width 0.5) (layer "B.Cu") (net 7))
 (segment (start 146.9305 113.726) (end 147.6815 112.975) (width 0.5) (layer "B.Cu") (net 7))
 (segment (start 142.24 114.3) (end 145.0705 114.3) (width 0.5) (layer "F.Cu") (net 6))
 (segment (start 149.586 112.975) (end 150.271 113.66) (width 0.5) (layer "F.Cu") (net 6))
 (segment (start 146.3955 112.975) (end 149.586 112.975) (width 0.5) (layer "F.Cu") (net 6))
 (segment (start 145.0705 114.3) (end 146.3955 112.975) (width 0.5) (layer "F.Cu") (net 6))
 (segment (start 143.5315 114.3) (end 145.0555 112.776) (width 0.5) (layer "B.Cu") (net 6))
 (segment (start 149.156 114.3) (end 148.98 114.476) (width 0.5) (layer "B.Cu") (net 6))
 (segment (start 142.24 114.3) (end 143.5315 114.3) (width 0.5) (layer "B.Cu") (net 6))
 (segment (start 145.972 114.476) (end 145.0555 113.5595) (width 0.5) (layer "B.Cu") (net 6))
 (segment (start 148.98 114.476) (end 145.972 114.476) (width 0.5) (layer "B.Cu") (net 6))
 (segment (start 145.0555 113.5595) (end 145.0555 112.776) (width 0.5) (layer "B.Cu") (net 6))
 (segment (start 149.858 112.173) (end 150.271 111.76) (width 0.5) (layer "F.Cu") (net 5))
 (segment (start 146.6955 112.173) (end 149.858 112.173) (width 0.5) (layer "F.Cu") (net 5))
 (segment (start 144.7585 111.76) (end 145.5205 110.998) (width 0.5) (layer "F.Cu") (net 5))
 (segment (start 142.24 111.76) (end 144.7585 111.76) (width 0.5) (layer "F.Cu") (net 5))
 (segment (start 145.5205 110.998) (end 146.6955 112.173) (width 0.5) (layer "F.Cu") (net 5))
 (segment (start 143.002 110.998) (end 142.24 111.76) (width 0.5) (layer "B.Cu") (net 5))
 (segment (start 149.606 110.998) (end 143.002 110.998) (width 0.5) (layer "B.Cu") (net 5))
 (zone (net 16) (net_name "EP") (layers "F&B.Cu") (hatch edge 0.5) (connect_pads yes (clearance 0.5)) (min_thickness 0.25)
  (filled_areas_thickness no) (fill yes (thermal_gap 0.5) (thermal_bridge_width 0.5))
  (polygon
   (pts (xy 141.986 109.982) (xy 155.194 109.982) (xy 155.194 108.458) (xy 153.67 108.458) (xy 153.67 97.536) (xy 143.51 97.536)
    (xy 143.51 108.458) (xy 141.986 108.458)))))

